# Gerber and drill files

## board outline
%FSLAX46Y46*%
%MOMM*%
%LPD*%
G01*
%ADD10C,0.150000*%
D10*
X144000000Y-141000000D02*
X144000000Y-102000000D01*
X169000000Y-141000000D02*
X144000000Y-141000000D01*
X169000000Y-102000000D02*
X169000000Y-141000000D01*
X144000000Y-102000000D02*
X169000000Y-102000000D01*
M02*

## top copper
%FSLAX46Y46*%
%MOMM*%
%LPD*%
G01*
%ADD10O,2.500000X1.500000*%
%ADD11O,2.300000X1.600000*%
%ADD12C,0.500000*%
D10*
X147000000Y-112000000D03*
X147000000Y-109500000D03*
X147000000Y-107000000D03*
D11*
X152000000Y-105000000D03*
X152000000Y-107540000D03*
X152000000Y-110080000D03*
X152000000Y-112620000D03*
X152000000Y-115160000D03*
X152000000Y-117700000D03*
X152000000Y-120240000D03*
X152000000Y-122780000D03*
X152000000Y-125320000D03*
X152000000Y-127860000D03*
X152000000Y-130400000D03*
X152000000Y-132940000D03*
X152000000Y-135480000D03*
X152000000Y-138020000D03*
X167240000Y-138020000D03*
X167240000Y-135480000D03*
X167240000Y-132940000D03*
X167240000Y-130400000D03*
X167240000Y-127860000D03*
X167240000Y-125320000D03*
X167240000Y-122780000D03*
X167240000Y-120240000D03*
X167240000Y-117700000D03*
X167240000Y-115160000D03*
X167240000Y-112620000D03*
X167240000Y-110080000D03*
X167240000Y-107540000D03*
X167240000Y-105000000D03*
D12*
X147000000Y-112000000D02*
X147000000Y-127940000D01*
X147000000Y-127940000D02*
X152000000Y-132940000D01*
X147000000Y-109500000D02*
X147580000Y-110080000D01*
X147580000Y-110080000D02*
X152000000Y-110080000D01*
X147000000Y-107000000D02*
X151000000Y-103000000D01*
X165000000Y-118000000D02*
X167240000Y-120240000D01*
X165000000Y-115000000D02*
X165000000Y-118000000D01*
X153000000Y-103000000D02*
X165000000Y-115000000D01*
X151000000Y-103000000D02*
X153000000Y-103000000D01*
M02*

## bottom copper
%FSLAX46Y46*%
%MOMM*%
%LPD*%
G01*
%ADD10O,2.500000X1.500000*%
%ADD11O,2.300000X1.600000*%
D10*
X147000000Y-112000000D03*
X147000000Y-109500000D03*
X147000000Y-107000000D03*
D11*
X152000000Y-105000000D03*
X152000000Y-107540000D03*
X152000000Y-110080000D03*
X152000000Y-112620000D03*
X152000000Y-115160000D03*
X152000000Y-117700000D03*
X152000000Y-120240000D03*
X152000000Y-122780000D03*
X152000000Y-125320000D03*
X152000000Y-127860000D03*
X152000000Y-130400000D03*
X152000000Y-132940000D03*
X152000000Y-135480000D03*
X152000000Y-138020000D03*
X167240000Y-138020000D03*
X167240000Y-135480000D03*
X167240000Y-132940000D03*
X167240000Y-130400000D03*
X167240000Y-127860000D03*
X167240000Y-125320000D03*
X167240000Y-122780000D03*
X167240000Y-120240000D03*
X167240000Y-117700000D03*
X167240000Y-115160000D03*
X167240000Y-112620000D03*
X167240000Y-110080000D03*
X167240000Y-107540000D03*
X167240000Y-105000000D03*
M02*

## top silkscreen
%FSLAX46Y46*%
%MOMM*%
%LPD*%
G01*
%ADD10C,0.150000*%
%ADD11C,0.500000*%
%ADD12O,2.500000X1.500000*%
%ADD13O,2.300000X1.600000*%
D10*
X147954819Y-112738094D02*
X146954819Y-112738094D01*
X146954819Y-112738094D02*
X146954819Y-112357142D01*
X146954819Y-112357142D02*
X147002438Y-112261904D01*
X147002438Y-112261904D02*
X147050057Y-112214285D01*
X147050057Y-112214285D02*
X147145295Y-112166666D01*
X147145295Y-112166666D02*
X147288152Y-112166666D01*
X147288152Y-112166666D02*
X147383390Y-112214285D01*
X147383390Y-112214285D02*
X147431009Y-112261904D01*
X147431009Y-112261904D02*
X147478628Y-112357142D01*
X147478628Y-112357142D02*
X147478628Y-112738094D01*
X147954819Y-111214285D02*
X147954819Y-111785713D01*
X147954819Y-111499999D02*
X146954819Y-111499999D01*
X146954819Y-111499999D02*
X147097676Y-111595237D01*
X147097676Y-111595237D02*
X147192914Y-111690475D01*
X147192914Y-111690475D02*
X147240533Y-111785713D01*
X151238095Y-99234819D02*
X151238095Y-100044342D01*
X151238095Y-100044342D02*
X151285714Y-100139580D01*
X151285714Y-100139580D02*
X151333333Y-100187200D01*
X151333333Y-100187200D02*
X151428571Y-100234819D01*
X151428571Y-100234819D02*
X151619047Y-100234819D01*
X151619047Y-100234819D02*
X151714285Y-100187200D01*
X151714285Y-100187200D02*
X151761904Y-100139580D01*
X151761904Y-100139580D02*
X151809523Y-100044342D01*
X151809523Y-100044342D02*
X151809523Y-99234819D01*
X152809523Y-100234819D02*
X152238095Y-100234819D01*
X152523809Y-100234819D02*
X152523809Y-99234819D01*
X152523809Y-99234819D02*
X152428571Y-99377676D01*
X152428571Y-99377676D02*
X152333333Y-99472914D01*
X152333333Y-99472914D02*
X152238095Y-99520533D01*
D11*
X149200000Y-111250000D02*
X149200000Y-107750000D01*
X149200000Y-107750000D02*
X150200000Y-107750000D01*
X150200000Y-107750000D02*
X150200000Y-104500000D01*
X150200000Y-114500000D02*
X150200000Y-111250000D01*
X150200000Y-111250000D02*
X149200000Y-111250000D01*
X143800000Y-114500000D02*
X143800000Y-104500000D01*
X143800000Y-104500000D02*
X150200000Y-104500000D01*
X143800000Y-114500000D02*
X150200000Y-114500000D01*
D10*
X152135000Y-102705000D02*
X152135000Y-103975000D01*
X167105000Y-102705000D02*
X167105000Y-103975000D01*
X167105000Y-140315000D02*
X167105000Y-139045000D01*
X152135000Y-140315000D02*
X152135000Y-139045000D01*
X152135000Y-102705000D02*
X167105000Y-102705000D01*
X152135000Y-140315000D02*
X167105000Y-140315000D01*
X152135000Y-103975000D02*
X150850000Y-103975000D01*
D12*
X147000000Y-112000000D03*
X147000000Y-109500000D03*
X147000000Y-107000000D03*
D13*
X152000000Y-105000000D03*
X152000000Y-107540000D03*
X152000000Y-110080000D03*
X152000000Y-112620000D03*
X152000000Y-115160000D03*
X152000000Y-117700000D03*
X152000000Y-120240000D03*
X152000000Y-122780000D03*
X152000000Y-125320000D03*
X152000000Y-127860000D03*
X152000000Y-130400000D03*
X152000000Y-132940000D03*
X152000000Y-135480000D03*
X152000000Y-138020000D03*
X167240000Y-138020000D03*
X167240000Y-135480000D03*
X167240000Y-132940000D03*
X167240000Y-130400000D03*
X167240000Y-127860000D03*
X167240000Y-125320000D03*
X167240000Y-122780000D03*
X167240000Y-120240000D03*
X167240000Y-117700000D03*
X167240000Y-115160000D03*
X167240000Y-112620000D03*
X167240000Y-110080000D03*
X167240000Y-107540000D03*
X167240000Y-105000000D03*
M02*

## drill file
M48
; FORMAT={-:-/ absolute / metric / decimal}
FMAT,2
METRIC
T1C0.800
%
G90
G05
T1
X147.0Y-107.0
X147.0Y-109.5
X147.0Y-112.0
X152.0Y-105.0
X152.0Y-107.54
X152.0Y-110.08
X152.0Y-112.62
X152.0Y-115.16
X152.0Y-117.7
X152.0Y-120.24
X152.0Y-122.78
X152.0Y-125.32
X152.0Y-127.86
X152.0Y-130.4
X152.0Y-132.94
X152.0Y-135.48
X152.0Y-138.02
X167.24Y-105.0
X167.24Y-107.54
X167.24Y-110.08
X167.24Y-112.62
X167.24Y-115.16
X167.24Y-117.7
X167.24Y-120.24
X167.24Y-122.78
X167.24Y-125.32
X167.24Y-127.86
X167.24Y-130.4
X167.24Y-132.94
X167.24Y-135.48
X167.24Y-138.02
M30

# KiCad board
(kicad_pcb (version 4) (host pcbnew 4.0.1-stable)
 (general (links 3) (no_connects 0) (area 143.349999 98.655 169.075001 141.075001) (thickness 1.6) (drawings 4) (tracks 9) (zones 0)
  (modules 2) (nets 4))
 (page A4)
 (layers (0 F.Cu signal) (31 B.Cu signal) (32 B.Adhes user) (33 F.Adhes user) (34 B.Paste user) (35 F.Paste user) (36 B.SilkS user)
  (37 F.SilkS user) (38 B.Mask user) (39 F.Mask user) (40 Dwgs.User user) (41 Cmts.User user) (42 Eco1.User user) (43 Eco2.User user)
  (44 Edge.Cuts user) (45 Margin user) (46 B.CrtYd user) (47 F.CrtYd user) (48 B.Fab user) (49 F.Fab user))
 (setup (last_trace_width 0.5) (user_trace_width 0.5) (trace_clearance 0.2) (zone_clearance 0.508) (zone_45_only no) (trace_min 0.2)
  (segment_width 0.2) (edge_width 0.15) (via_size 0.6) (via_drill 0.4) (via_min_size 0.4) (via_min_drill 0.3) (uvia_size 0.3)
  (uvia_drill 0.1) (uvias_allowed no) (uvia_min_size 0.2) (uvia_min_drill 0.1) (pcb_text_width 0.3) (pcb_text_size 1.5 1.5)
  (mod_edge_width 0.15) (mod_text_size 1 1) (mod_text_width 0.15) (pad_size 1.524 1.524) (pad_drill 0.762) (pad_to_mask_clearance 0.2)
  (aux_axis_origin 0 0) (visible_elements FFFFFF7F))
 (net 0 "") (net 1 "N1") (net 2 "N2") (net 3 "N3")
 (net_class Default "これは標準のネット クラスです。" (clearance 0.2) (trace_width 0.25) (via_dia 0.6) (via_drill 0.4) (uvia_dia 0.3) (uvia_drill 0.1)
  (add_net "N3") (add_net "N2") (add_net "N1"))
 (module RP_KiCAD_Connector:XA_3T (layer F.Cu) (at 147 112 90)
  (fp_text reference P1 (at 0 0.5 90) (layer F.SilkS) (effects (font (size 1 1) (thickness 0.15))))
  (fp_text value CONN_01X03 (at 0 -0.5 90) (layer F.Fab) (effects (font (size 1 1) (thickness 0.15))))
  (fp_line (start 0.75 2.2) (end 4.25 2.2) (layer F.SilkS) (width 0.5))
  (fp_line (start 4.25 2.2) (end 4.25 3.2) (layer F.SilkS) (width 0.5))
  (fp_line (start 4.25 3.2) (end 7.5 3.2) (layer F.SilkS) (width 0.5))
  (fp_line (start -2.5 3.2) (end 0.75 3.2) (layer F.SilkS) (width 0.5))
  (fp_line (start 0.75 3.2) (end 0.75 2.2) (layer F.SilkS) (width 0.5))
  (fp_line (start -2.5 -3.2) (end 7.5 -3.2) (layer F.SilkS) (width 0.5))
  (fp_line (start 7.5 -3.2) (end 7.5 3.2) (layer F.SilkS) (width 0.5))
  (fp_line (start -2.5 -3.2) (end -2.5 3.2) (layer F.SilkS) (width 0.5))
  (pad 3 thru_hole oval (at 0 0 90) (size 1.5 2.5) (drill 0.8) (layers *.Cu *.Mask F.SilkS) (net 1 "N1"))
  (pad 2 thru_hole oval (at 2.5 0 90) (size 1.5 2.5) (drill 0.8) (layers *.Cu *.Mask F.SilkS) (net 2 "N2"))
  (pad 1 thru_hole oval (at 5 0 90) (size 1.5 2.5) (drill 0.8) (layers *.Cu *.Mask F.SilkS) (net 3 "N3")))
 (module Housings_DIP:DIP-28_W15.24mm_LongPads (layer F.Cu) (at 152 105)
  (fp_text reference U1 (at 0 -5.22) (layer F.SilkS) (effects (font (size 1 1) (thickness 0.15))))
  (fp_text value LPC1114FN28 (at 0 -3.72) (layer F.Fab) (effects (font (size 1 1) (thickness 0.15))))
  (fp_line (start 0.135 -2.295) (end 0.135 -1.025) (layer F.SilkS) (width 0.15))
  (fp_line (start 15.105 -2.295) (end 15.105 -1.025) (layer F.SilkS) (width 0.15))
  (fp_line (start 15.105 35.315) (end 15.105 34.045) (layer F.SilkS) (width 0.15))
  (fp_line (start 0.135 35.315) (end 0.135 34.045) (layer F.SilkS) (width 0.15))
  (fp_line (start 0.135 -2.295) (end 15.105 -2.295) (layer F.SilkS) (width 0.15))
  (fp_line (start 0.135 35.315) (end 15.105 35.315) (layer F.SilkS) (width 0.15))
  (fp_line (start 0.135 -1.025) (end -1.15 -1.025) (layer F.SilkS) (width 0.15))
  (pad 1 thru_hole oval (at 0 0) (size 2.3 1.6) (drill 0.8) (layers *.Cu *.Mask F.SilkS))
  (pad 2 thru_hole oval (at 0 2.54) (size 2.3 1.6) (drill 0.8) (layers *.Cu *.Mask F.SilkS))
  (pad 3 thru_hole oval (at 0 5.08) (size 2.3 1.6) (drill 0.8) (layers *.Cu *.Mask F.SilkS) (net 2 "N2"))
  (pad 4 thru_hole oval (at 0 7.62) (size 2.3 1.6) (drill 0.8) (layers *.Cu *.Mask F.SilkS))
  (pad 5 thru_hole oval (at 0 10.16) (size 2.3 1.6) (drill 0.8) (layers *.Cu *.Mask F.SilkS))
  (pad 6 thru_hole oval (at 0 12.7) (size 2.3 1.6) (drill 0.8) (layers *.Cu *.Mask F.SilkS))
  (pad 7 thru_hole oval (at 0 15.24) (size 2.3 1.6) (drill 0.8) (layers *.Cu *.Mask F.SilkS))
  (pad 8 thru_hole oval (at 0 17.78) (size 2.3 1.6) (drill 0.8) (layers *.Cu *.Mask F.SilkS))
  (pad 9 thru_hole oval (at 0 20.32) (size 2.3 1.6) (drill 0.8) (layers *.Cu *.Mask F.SilkS))
  (pad 10 thru_hole oval (at 0 22.86) (size 2.3 1.6) (drill 0.8) (layers *.Cu *.Mask F.SilkS))
  (pad 11 thru_hole oval (at 0 25.4) (size 2.3 1.6) (drill 0.8) (layers *.Cu *.Mask F.SilkS))
  (pad 12 thru_hole oval (at 0 27.94) (size 2.3 1.6) (drill 0.8) (layers *.Cu *.Mask F.SilkS) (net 1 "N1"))
  (pad 13 thru_hole oval (at 0 30.48) (size 2.3 1.6) (drill 0.8) (layers *.Cu *.Mask F.SilkS))
  (pad 14 thru_hole oval (at 0 33.02) (size 2.3 1.6) (drill 0.8) (layers *.Cu *.Mask F.SilkS))
  (pad 15 thru_hole oval (at 15.24 33.02) (size 2.3 1.6) (drill 0.8) (layers *.Cu *.Mask F.SilkS))
  (pad 16 thru_hole oval (at 15.24 30.48) (size 2.3 1.6) (drill 0.8) (layers *.Cu *.Mask F.SilkS))
  (pad 17 thru_hole oval (at 15.24 27.94) (size 2.3 1.6) (drill 0.8) (layers *.Cu *.Mask F.SilkS))
  (pad 18 thru_hole oval (at 15.24 25.4) (size 2.3 1.6) (drill 0.8) (layers *.Cu *.Mask F.SilkS))
  (pad 19 thru_hole oval (at 15.24 22.86) (size 2.3 1.6) (drill 0.8) (layers *.Cu *.Mask F.SilkS))
  (pad 20 thru_hole oval (at 15.24 20.32) (size 2.3 1.6) (drill 0.8) (layers *.Cu *.Mask F.SilkS))
  (pad 21 thru_hole oval (at 15.24 17.78) (size 2.3 1.6) (drill 0.8) (layers *.Cu *.Mask F.SilkS))
  (pad 22 thru_hole oval (at 15.24 15.24) (size 2.3 1.6) (drill 0.8) (layers *.Cu *.Mask F.SilkS) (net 3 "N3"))
  (pad 23 thru_hole oval (at 15.24 12.7) (size 2.3 1.6) (drill 0.8) (layers *.Cu *.Mask F.SilkS))
  (pad 24 thru_hole oval (at 15.24 10.16) (size 2.3 1.6) (drill 0.8) (layers *.Cu *.Mask F.SilkS))
  (pad 25 thru_hole oval (at 15.24 7.62) (size 2.3 1.6) (drill 0.8) (layers *.Cu *.Mask F.SilkS))
  (pad 26 thru_hole oval (at 15.24 5.08) (size 2.3 1.6) (drill 0.8) (layers *.Cu *.Mask F.SilkS))
  (pad 27 thru_hole oval (at 15.24 2.54) (size 2.3 1.6) (drill 0.8) (layers *.Cu *.Mask F.SilkS))
  (pad 28 thru_hole oval (at 15.24 0) (size 2.3 1.6) (drill 0.8) (layers *.Cu *.Mask F.SilkS)))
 (gr_line (start 144 141) (end 144 102) (angle 90) (layer Edge.Cuts) (width 0.15))
 (gr_line (start 169 141) (end 144 141) (angle 90) (layer Edge.Cuts) (width 0.15))
 (gr_line (start 169 102) (end 169 141) (angle 90) (layer Edge.Cuts) (width 0.15))
 (gr_line (start 144 102) (end 169 102) (angle 90) (layer Edge.Cuts) (width 0.15))
 (segment (start 147 112) (end 147 127.94) (width 0.5) (layer F.Cu) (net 1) (status 400000))
 (segment (start 147 127.94) (end 152 132.94) (width 0.5) (layer F.Cu) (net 1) (status 800000))
 (segment (start 147 109.5) (end 147.58 110.08) (width 0.5) (layer F.Cu) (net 2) (status C00000))
 (segment (start 147.58 110.08) (end 152 110.08) (width 0.5) (layer F.Cu) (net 2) (status C00000))
 (segment (start 147 107) (end 151 103) (width 0.5) (layer F.Cu) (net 3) (status 400000))
 (segment (start 165 118) (end 167.24 120.24) (width 0.5) (layer F.Cu) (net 3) (status 800000))
 (segment (start 165 115) (end 165 118) (width 0.5) (layer F.Cu) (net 3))
 (segment (start 153 103) (end 165 115) (width 0.5) (layer F.Cu) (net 3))
 (segment (start 151 103) (end 153 103) (width 0.5) (layer F.Cu) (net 3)))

